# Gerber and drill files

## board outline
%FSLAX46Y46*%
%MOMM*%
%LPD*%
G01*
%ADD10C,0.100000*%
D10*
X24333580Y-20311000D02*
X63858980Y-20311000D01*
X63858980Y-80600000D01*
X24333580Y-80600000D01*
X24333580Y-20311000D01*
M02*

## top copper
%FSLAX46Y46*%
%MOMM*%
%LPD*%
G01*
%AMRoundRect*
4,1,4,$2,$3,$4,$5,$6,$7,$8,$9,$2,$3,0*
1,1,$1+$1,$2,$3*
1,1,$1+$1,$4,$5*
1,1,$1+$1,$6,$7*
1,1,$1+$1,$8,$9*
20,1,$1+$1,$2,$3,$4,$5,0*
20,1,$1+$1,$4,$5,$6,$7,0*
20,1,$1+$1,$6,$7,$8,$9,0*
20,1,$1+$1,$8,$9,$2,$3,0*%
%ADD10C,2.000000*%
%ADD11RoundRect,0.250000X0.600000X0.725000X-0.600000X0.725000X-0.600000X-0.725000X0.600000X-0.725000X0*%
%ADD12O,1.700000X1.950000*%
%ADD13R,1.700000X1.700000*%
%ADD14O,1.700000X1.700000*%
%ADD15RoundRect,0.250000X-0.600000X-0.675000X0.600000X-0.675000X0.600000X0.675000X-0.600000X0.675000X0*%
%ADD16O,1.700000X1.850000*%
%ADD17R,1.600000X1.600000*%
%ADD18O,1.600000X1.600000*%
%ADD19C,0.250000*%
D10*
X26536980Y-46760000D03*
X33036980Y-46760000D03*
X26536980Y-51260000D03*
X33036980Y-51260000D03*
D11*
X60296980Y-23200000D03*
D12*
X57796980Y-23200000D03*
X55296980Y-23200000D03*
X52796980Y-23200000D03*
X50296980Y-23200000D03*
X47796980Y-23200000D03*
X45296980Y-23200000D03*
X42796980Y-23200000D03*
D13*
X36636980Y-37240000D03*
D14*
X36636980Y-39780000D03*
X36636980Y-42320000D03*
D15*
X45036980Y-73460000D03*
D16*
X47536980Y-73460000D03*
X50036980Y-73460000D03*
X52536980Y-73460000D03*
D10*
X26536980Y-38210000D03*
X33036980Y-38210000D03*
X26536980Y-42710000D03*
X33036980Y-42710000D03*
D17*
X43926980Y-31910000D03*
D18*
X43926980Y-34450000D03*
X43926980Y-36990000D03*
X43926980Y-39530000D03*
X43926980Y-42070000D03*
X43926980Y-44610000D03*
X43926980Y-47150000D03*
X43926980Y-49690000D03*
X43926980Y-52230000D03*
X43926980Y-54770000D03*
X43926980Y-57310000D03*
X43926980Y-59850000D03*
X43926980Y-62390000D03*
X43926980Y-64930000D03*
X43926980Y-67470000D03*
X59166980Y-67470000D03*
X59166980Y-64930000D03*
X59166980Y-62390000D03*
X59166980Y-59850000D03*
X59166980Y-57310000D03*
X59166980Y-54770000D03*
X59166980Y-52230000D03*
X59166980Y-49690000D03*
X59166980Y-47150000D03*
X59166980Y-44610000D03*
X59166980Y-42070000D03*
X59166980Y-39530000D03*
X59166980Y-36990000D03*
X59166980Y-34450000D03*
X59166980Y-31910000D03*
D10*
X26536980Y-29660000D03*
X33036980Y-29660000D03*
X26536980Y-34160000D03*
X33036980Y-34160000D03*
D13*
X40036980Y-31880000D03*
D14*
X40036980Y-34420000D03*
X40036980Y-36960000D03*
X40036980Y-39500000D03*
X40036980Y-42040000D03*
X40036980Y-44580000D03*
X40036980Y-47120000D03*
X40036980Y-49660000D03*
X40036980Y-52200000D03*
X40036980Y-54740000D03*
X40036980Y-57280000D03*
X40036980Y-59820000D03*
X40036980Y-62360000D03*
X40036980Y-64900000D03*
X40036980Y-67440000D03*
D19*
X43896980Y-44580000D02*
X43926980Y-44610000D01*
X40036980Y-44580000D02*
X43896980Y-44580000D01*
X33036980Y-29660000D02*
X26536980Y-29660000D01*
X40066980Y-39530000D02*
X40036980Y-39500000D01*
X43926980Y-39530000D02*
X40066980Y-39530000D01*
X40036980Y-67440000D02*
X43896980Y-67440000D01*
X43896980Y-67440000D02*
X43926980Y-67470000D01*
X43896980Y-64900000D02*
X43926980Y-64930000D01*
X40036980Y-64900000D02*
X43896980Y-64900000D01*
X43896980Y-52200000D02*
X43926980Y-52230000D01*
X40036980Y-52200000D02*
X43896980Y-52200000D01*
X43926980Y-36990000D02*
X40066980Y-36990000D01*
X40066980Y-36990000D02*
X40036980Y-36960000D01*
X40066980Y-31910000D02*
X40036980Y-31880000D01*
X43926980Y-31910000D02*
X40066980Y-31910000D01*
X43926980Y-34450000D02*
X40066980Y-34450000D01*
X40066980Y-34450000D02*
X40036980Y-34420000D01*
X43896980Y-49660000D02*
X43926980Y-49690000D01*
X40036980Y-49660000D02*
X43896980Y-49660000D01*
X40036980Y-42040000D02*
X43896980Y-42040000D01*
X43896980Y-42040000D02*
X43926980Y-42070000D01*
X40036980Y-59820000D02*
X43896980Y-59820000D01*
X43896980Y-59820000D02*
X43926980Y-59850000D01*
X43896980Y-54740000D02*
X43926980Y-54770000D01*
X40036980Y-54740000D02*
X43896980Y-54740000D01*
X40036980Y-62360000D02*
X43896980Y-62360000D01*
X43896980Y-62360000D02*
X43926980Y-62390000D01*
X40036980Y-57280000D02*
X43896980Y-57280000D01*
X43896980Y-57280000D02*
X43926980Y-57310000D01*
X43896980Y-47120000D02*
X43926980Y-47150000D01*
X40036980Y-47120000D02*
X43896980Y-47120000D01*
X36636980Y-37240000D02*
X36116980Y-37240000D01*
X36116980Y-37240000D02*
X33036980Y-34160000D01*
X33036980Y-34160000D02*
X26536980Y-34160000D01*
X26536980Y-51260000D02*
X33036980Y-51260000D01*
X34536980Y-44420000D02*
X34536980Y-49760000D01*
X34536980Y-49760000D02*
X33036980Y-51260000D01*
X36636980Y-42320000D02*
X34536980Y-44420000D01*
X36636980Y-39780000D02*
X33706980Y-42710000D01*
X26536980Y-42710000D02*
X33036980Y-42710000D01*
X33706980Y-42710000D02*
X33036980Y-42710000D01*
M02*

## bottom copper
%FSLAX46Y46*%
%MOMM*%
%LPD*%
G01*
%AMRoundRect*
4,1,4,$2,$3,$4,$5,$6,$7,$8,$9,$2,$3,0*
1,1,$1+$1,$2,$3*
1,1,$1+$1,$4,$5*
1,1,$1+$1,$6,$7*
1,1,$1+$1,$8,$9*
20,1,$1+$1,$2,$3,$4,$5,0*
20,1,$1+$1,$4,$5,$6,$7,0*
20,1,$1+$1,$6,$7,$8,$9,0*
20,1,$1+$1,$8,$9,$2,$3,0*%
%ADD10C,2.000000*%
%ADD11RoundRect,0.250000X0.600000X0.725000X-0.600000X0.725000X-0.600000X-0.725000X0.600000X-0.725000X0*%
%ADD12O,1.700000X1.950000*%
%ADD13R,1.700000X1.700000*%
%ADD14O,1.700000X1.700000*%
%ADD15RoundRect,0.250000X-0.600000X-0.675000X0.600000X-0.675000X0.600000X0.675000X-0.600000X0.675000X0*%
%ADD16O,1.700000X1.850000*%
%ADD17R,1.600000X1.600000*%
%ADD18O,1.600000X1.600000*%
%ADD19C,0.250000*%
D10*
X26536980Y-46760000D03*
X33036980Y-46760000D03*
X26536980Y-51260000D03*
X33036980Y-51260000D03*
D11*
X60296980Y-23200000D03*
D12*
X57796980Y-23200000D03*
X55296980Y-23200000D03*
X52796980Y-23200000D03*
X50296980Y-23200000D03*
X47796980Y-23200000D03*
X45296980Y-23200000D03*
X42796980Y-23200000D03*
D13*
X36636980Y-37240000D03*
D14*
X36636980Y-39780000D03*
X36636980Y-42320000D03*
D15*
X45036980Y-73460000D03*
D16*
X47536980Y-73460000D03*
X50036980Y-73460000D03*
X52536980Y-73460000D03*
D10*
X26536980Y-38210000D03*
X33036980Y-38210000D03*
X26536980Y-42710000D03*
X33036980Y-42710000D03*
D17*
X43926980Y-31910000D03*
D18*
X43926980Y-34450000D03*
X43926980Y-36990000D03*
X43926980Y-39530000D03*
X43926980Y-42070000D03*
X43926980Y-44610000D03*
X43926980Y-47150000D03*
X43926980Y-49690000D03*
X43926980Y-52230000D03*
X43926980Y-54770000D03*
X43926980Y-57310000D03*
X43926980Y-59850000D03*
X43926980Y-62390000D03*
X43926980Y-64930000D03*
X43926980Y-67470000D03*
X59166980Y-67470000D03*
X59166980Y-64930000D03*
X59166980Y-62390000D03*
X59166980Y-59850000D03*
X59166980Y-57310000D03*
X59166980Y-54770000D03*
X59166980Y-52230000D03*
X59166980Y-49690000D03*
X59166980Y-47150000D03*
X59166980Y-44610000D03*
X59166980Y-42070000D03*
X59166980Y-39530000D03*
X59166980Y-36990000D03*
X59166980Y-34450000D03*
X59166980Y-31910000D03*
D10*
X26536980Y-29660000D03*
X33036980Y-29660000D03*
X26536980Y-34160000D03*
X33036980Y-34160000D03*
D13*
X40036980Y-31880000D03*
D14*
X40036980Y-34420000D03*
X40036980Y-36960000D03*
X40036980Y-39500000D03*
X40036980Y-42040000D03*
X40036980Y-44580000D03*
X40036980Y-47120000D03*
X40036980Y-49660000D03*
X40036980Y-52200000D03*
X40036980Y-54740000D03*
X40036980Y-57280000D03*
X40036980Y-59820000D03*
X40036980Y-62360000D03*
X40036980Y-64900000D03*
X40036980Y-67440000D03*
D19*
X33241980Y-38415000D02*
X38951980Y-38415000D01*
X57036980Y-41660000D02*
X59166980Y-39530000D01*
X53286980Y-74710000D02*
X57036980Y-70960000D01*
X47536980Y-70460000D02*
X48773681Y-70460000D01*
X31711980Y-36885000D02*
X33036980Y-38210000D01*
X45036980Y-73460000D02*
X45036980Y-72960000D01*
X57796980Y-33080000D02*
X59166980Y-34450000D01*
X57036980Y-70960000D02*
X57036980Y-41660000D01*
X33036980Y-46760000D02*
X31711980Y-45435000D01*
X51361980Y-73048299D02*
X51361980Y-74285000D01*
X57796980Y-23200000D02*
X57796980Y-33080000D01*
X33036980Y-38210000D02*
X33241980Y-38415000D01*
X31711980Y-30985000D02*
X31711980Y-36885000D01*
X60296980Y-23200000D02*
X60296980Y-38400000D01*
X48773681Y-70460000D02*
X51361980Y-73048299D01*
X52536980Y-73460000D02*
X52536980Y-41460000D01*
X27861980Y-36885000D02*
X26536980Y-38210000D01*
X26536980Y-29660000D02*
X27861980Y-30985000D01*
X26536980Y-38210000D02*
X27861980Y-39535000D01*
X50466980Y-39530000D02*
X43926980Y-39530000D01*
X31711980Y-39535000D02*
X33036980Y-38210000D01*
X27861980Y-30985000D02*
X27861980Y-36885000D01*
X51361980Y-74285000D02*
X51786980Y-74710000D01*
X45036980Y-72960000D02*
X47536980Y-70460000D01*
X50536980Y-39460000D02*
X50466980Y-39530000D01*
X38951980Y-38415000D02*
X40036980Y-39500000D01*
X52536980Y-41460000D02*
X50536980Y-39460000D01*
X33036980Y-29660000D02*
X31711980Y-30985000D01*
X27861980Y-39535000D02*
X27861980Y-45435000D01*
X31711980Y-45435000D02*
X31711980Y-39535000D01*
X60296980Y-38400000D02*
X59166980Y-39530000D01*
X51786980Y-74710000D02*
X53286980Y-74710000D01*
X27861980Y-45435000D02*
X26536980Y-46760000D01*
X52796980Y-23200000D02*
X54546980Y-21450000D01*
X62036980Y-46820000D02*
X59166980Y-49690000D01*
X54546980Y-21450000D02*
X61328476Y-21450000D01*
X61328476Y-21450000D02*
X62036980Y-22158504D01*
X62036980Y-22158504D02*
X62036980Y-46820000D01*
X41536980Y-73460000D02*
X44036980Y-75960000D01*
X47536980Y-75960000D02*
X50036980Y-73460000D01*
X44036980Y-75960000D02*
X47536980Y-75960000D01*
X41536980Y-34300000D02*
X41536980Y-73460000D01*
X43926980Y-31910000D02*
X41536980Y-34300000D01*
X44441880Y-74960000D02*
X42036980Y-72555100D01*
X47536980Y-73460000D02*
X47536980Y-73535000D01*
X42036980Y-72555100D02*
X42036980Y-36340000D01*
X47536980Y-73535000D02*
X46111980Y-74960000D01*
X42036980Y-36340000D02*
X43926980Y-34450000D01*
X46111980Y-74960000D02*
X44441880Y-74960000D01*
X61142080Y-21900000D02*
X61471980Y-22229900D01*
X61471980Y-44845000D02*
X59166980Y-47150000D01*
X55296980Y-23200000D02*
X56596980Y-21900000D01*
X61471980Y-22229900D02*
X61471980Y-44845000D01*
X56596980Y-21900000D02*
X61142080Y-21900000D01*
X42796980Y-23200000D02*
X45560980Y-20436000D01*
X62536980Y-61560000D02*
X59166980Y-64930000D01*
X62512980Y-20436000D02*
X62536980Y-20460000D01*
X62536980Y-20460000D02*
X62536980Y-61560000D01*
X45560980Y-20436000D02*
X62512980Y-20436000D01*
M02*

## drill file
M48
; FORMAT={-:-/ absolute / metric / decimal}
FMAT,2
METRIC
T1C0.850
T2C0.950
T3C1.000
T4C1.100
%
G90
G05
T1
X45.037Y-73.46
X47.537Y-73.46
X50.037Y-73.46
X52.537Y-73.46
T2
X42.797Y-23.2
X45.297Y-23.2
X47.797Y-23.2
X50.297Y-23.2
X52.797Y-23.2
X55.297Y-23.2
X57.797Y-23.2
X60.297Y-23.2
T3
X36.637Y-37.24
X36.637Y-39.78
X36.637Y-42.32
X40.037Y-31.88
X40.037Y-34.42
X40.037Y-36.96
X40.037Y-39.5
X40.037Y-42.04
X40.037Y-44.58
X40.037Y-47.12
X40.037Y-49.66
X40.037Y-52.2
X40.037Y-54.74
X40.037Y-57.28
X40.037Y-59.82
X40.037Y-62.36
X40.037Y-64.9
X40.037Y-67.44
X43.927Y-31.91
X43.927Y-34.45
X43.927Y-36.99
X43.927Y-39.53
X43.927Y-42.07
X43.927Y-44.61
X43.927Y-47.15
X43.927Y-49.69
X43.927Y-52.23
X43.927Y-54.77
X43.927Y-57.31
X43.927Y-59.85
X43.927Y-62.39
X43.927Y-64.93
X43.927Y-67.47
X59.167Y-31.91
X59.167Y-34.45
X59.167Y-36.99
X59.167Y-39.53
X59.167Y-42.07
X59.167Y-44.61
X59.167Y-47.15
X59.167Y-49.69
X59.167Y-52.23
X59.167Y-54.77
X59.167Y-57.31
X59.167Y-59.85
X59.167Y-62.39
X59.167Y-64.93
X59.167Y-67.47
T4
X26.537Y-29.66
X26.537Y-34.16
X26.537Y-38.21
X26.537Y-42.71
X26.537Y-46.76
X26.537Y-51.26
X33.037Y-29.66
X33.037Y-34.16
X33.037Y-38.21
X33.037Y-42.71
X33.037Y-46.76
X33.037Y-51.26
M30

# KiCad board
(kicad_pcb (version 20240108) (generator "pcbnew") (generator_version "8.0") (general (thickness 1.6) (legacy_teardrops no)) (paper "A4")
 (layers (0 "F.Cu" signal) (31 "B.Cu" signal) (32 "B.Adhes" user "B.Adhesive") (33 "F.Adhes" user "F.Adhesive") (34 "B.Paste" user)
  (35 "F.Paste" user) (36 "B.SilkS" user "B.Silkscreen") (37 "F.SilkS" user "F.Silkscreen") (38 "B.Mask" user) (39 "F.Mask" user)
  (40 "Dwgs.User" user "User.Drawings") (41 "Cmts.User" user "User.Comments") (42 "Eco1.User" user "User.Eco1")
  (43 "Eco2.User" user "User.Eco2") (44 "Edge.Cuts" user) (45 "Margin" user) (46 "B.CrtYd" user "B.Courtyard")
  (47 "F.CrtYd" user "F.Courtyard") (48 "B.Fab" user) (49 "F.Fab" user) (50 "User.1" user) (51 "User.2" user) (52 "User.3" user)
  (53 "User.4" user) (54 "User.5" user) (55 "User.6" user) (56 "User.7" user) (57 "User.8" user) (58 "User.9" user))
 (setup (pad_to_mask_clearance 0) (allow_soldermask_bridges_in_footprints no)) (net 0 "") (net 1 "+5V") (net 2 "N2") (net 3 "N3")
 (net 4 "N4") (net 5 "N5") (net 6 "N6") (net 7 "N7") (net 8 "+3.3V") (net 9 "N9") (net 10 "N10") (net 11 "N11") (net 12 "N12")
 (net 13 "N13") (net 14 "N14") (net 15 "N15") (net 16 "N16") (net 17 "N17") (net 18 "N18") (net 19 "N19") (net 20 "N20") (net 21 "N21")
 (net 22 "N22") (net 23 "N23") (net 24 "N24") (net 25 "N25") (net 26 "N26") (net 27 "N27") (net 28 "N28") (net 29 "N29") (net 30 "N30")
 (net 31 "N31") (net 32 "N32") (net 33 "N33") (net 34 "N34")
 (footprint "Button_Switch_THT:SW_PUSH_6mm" (layer "F.Cu") (at 26.53698 46.76)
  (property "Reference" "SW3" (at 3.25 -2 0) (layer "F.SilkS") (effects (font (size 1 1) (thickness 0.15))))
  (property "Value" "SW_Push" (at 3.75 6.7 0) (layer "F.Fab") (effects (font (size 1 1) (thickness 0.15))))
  (pad "1" thru_hole circle (at 0 0 90) (size 2 2) (drill 1.1) (layers "*.Cu" "*.Mask") (remove_unused_layers no) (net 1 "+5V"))
  (pad "1" thru_hole circle (at 6.5 0 90) (size 2 2) (drill 1.1) (layers "*.Cu" "*.Mask") (remove_unused_layers no) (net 1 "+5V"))
  (pad "2" thru_hole circle (at 0 4.5 90) (size 2 2) (drill 1.1) (layers "*.Cu" "*.Mask") (remove_unused_layers no) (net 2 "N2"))
  (pad "2" thru_hole circle (at 6.5 4.5 90) (size 2 2) (drill 1.1) (layers "*.Cu" "*.Mask") (remove_unused_layers no) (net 2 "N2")))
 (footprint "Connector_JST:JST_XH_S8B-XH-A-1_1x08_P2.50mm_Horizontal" (layer "F.Cu") (at 60.29698 23.2 180)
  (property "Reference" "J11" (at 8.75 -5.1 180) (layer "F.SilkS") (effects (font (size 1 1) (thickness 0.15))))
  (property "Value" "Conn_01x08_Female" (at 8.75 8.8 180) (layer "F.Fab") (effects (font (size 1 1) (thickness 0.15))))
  (pad "1" thru_hole roundrect (at 0 0 180) (size 1.7 1.95) (drill 0.95) (layers "*.Cu" "*.Mask") (remove_unused_layers no)
   (roundrect_rratio 0.147059) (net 1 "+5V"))
  (pad "2" thru_hole oval (at 2.5 0 180) (size 1.7 1.95) (drill 0.95) (layers "*.Cu" "*.Mask") (remove_unused_layers no) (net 1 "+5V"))
  (pad "3" thru_hole oval (at 5 0 180) (size 1.7 1.95) (drill 0.95) (layers "*.Cu" "*.Mask") (remove_unused_layers no) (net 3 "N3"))
  (pad "4" thru_hole oval (at 7.5 0 180) (size 1.7 1.95) (drill 0.95) (layers "*.Cu" "*.Mask") (remove_unused_layers no) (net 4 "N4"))
  (pad "5" thru_hole oval (at 10 0 180) (size 1.7 1.95) (drill 0.95) (layers "*.Cu" "*.Mask") (remove_unused_layers no) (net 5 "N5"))
  (pad "6" thru_hole oval (at 12.5 0 180) (size 1.7 1.95) (drill 0.95) (layers "*.Cu" "*.Mask") (remove_unused_layers no) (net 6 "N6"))
  (pad "7" thru_hole oval (at 15 0 180) (size 1.7 1.95) (drill 0.95) (layers "*.Cu" "*.Mask") (remove_unused_layers no) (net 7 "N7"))
  (pad "8" thru_hole oval (at 17.5 0 180) (size 1.7 1.95) (drill 0.95) (layers "*.Cu" "*.Mask") (remove_unused_layers no) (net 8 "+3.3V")))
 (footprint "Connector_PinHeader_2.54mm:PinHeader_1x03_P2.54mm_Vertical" (layer "F.Cu") (at 36.63698 37.24)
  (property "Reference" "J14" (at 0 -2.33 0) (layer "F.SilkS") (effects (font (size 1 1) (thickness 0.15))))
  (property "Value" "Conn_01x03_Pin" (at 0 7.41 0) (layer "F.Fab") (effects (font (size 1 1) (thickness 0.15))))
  (pad "1" thru_hole rect (at 0 0) (size 1.7 1.7) (drill 1) (layers "*.Cu" "*.Mask") (remove_unused_layers no) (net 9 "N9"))
  (pad "2" thru_hole oval (at 0 2.54) (size 1.7 1.7) (drill 1) (layers "*.Cu" "*.Mask") (remove_unused_layers no) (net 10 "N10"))
  (pad "3" thru_hole oval (at 0 5.08) (size 1.7 1.7) (drill 1) (layers "*.Cu" "*.Mask") (remove_unused_layers no) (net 2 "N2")))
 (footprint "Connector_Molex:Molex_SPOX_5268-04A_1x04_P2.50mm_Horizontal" (layer "F.Cu") (at 45.03698 73.46)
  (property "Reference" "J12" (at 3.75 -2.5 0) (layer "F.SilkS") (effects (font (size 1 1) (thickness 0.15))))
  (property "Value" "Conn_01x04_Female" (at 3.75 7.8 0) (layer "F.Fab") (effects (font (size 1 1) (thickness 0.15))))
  (pad "1" thru_hole roundrect (at 0 0) (size 1.7 1.85) (drill 0.85) (layers "*.Cu" "*.Mask") (remove_unused_layers no)
   (roundrect_rratio 0.147059) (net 1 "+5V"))
  (pad "2" thru_hole oval (at 2.5 0) (size 1.7 1.85) (drill 0.85) (layers "*.Cu" "*.Mask") (remove_unused_layers no) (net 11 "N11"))
  (pad "3" thru_hole oval (at 5 0) (size 1.7 1.85) (drill 0.85) (layers "*.Cu" "*.Mask") (remove_unused_layers no) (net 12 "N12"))
  (pad "4" thru_hole oval (at 7.5 0) (size 1.7 1.85) (drill 0.85) (layers "*.Cu" "*.Mask") (remove_unused_layers no) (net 1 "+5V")))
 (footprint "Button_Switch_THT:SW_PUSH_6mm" (layer "F.Cu") (at 26.53698 38.21)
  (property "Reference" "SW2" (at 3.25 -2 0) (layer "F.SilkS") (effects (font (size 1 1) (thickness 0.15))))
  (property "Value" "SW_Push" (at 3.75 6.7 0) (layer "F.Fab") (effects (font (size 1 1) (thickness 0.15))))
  (pad "1" thru_hole circle (at 0 0 90) (size 2 2) (drill 1.1) (layers "*.Cu" "*.Mask") (remove_unused_layers no) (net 1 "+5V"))
  (pad "1" thru_hole circle (at 6.5 0 90) (size 2 2) (drill 1.1) (layers "*.Cu" "*.Mask") (remove_unused_layers no) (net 1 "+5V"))
  (pad "2" thru_hole circle (at 0 4.5 90) (size 2 2) (drill 1.1) (layers "*.Cu" "*.Mask") (remove_unused_layers no) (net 10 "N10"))
  (pad "2" thru_hole circle (at 6.5 4.5 90) (size 2 2) (drill 1.1) (layers "*.Cu" "*.Mask") (remove_unused_layers no) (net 10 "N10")))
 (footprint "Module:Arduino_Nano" (layer "F.Cu") (at 43.92698 31.91)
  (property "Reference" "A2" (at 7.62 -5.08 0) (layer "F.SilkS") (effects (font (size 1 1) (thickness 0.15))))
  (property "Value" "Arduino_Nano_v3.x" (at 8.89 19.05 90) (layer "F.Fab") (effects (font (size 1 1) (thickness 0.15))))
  (pad "1" thru_hole rect (at 0 0) (size 1.6 1.6) (drill 1) (layers "*.Cu" "*.Mask") (remove_unused_layers no) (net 12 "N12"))
  (pad "2" thru_hole oval (at 0 2.54) (size 1.6 1.6) (drill 1) (layers "*.Cu" "*.Mask") (remove_unused_layers no) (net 11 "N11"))
  (pad "3" thru_hole oval (at 0 5.08) (size 1.6 1.6) (drill 1) (layers "*.Cu" "*.Mask") (remove_unused_layers no) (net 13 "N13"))
  (pad "4" thru_hole oval (at 0 7.62) (size 1.6 1.6) (drill 1) (layers "*.Cu" "*.Mask") (remove_unused_layers no) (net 1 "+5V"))
  (pad "5" thru_hole oval (at 0 10.16) (size 1.6 1.6) (drill 1) (layers "*.Cu" "*.Mask") (remove_unused_layers no) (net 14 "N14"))
  (pad "6" thru_hole oval (at 0 12.7) (size 1.6 1.6) (drill 1) (layers "*.Cu" "*.Mask") (remove_unused_layers no) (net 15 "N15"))
  (pad "7" thru_hole oval (at 0 15.24) (size 1.6 1.6) (drill 1) (layers "*.Cu" "*.Mask") (remove_unused_layers no) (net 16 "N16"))
  (pad "8" thru_hole oval (at 0 17.78) (size 1.6 1.6) (drill 1) (layers "*.Cu" "*.Mask") (remove_unused_layers no) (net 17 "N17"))
  (pad "9" thru_hole oval (at 0 20.32) (size 1.6 1.6) (drill 1) (layers "*.Cu" "*.Mask") (remove_unused_layers no) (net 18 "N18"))
  (pad "10" thru_hole oval (at 0 22.86) (size 1.6 1.6) (drill 1) (layers "*.Cu" "*.Mask") (remove_unused_layers no) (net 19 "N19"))
  (pad "11" thru_hole oval (at 0 25.4) (size 1.6 1.6) (drill 1) (layers "*.Cu" "*.Mask") (remove_unused_layers no) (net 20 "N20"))
  (pad "12" thru_hole oval (at 0 27.94) (size 1.6 1.6) (drill 1) (layers "*.Cu" "*.Mask") (remove_unused_layers no) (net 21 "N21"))
  (pad "13" thru_hole oval (at 0 30.48) (size 1.6 1.6) (drill 1) (layers "*.Cu" "*.Mask") (remove_unused_layers no) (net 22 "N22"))
  (pad "14" thru_hole oval (at 0 33.02) (size 1.6 1.6) (drill 1) (layers "*.Cu" "*.Mask") (remove_unused_layers no) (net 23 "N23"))
  (pad "15" thru_hole oval (at 0 35.56) (size 1.6 1.6) (drill 1) (layers "*.Cu" "*.Mask") (remove_unused_layers no) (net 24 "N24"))
  (pad "16" thru_hole oval (at 15.24 35.56) (size 1.6 1.6) (drill 1) (layers "*.Cu" "*.Mask") (remove_unused_layers no) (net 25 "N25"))
  (pad "17" thru_hole oval (at 15.24 33.02) (size 1.6 1.6) (drill 1) (layers "*.Cu" "*.Mask") (remove_unused_layers no) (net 8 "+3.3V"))
  (pad "18" thru_hole oval (at 15.24 30.48) (size 1.6 1.6) (drill 1) (layers "*.Cu" "*.Mask") (remove_unused_layers no) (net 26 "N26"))
  (pad "19" thru_hole oval (at 15.24 27.94) (size 1.6 1.6) (drill 1) (layers "*.Cu" "*.Mask") (remove_unused_layers no) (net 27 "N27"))
  (pad "20" thru_hole oval (at 15.24 25.4) (size 1.6 1.6) (drill 1) (layers "*.Cu" "*.Mask") (remove_unused_layers no) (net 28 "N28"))
  (pad "21" thru_hole oval (at 15.24 22.86) (size 1.6 1.6) (drill 1) (layers "*.Cu" "*.Mask") (remove_unused_layers no) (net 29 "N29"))
  (pad "22" thru_hole oval (at 15.24 20.32) (size 1.6 1.6) (drill 1) (layers "*.Cu" "*.Mask") (remove_unused_layers no) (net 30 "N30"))
  (pad "23" thru_hole oval (at 15.24 17.78) (size 1.6 1.6) (drill 1) (layers "*.Cu" "*.Mask") (remove_unused_layers no) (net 4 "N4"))
  (pad "24" thru_hole oval (at 15.24 15.24) (size 1.6 1.6) (drill 1) (layers "*.Cu" "*.Mask") (remove_unused_layers no) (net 3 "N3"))
  (pad "25" thru_hole oval (at 15.24 12.7) (size 1.6 1.6) (drill 1) (layers "*.Cu" "*.Mask") (remove_unused_layers no) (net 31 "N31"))
  (pad "26" thru_hole oval (at 15.24 10.16) (size 1.6 1.6) (drill 1) (layers "*.Cu" "*.Mask") (remove_unused_layers no) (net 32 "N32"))
  (pad "27" thru_hole oval (at 15.24 7.62) (size 1.6 1.6) (drill 1) (layers "*.Cu" "*.Mask") (remove_unused_layers no) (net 1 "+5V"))
  (pad "28" thru_hole oval (at 15.24 5.08) (size 1.6 1.6) (drill 1) (layers "*.Cu" "*.Mask") (remove_unused_layers no) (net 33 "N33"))
  (pad "29" thru_hole oval (at 15.24 2.54) (size 1.6 1.6) (drill 1) (layers "*.Cu" "*.Mask") (remove_unused_layers no) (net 1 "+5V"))
  (pad "30" thru_hole oval (at 15.24 0) (size 1.6 1.6) (drill 1) (layers "*.Cu" "*.Mask") (remove_unused_layers no) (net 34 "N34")))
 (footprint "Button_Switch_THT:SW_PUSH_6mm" (layer "F.Cu") (at 26.53698 29.66)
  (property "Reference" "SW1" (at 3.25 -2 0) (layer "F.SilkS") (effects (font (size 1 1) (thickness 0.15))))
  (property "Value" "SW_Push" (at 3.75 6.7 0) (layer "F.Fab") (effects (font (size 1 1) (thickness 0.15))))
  (pad "1" thru_hole circle (at 0 0 90) (size 2 2) (drill 1.1) (layers "*.Cu" "*.Mask") (remove_unused_layers no) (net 1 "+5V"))
  (pad "1" thru_hole circle (at 6.5 0 90) (size 2 2) (drill 1.1) (layers "*.Cu" "*.Mask") (remove_unused_layers no) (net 1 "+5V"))
  (pad "2" thru_hole circle (at 0 4.5 90) (size 2 2) (drill 1.1) (layers "*.Cu" "*.Mask") (remove_unused_layers no) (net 9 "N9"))
  (pad "2" thru_hole circle (at 6.5 4.5 90) (size 2 2) (drill 1.1) (layers "*.Cu" "*.Mask") (remove_unused_layers no) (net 9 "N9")))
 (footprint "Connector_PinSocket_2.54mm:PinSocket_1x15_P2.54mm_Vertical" (layer "F.Cu") (at 40.03698 31.88)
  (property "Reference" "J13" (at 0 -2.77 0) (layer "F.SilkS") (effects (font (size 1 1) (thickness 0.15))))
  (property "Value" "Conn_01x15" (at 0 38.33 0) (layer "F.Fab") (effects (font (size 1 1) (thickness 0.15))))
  (pad "1" thru_hole rect (at 0 0) (size 1.7 1.7) (drill 1) (layers "*.Cu" "*.Mask") (remove_unused_layers no) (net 12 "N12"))
  (pad "2" thru_hole oval (at 0 2.54) (size 1.7 1.7) (drill 1) (layers "*.Cu" "*.Mask") (remove_unused_layers no) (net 11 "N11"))
  (pad "3" thru_hole oval (at 0 5.08) (size 1.7 1.7) (drill 1) (layers "*.Cu" "*.Mask") (remove_unused_layers no) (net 13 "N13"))
  (pad "4" thru_hole oval (at 0 7.62) (size 1.7 1.7) (drill 1) (layers "*.Cu" "*.Mask") (remove_unused_layers no) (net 1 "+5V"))
  (pad "5" thru_hole oval (at 0 10.16) (size 1.7 1.7) (drill 1) (layers "*.Cu" "*.Mask") (remove_unused_layers no) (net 14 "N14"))
  (pad "6" thru_hole oval (at 0 12.7) (size 1.7 1.7) (drill 1) (layers "*.Cu" "*.Mask") (remove_unused_layers no) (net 15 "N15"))
  (pad "7" thru_hole oval (at 0 15.24) (size 1.7 1.7) (drill 1) (layers "*.Cu" "*.Mask") (remove_unused_layers no) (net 16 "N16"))
  (pad "8" thru_hole oval (at 0 17.78) (size 1.7 1.7) (drill 1) (layers "*.Cu" "*.Mask") (remove_unused_layers no) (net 17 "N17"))
  (pad "9" thru_hole oval (at 0 20.32) (size 1.7 1.7) (drill 1) (layers "*.Cu" "*.Mask") (remove_unused_layers no) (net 18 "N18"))
  (pad "10" thru_hole oval (at 0 22.86) (size 1.7 1.7) (drill 1) (layers "*.Cu" "*.Mask") (remove_unused_layers no) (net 19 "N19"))
  (pad "11" thru_hole oval (at 0 25.4) (size 1.7 1.7) (drill 1) (layers "*.Cu" "*.Mask") (remove_unused_layers no) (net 20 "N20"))
  (pad "12" thru_hole oval (at 0 27.94) (size 1.7 1.7) (drill 1) (layers "*.Cu" "*.Mask") (remove_unused_layers no) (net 21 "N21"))
  (pad "13" thru_hole oval (at 0 30.48) (size 1.7 1.7) (drill 1) (layers "*.Cu" "*.Mask") (remove_unused_layers no) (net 22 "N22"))
  (pad "14" thru_hole oval (at 0 33.02) (size 1.7 1.7) (drill 1) (layers "*.Cu" "*.Mask") (remove_unused_layers no) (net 23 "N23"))
  (pad "15" thru_hole oval (at 0 35.56) (size 1.7 1.7) (drill 1) (layers "*.Cu" "*.Mask") (remove_unused_layers no) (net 24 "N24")))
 (gr_rect (start 24.33358 20.311) (end 63.85898 80.6) (stroke (width 0.1) (type default)) (fill none) (layer "Edge.Cuts"))
 (segment (start 43.89698 44.58) (end 43.92698 44.61) (width 0.25) (layer "F.Cu") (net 15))
 (segment (start 40.03698 44.58) (end 43.89698 44.58) (width 0.25) (layer "F.Cu") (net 15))
 (segment (start 33.03698 29.66) (end 26.53698 29.66) (width 0.25) (layer "F.Cu") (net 1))
 (segment (start 40.06698 39.53) (end 40.03698 39.5) (width 0.25) (layer "F.Cu") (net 1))
 (segment (start 43.92698 39.53) (end 40.06698 39.53) (width 0.25) (layer "F.Cu") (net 1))
 (segment (start 33.24198 38.415) (end 38.95198 38.415) (width 0.25) (layer "B.Cu") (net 1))
 (segment (start 57.03698 41.66) (end 59.16698 39.53) (width 0.25) (layer "B.Cu") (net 1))
 (segment (start 53.28698 74.71) (end 57.03698 70.96) (width 0.25) (layer "B.Cu") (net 1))
 (segment (start 47.53698 70.46) (end 48.773681 70.46) (width 0.25) (layer "B.Cu") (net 1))
 (segment (start 31.71198 36.885) (end 33.03698 38.21) (width 0.25) (layer "B.Cu") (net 1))
 (segment (start 45.03698 73.46) (end 45.03698 72.96) (width 0.25) (layer "B.Cu") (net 1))
 (segment (start 57.79698 33.08) (end 59.16698 34.45) (width 0.25) (layer "B.Cu") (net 1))
 (segment (start 57.03698 70.96) (end 57.03698 41.66) (width 0.25) (layer "B.Cu") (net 1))
 (segment (start 33.03698 46.76) (end 31.71198 45.435) (width 0.25) (layer "B.Cu") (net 1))
 (segment (start 51.36198 73.048299) (end 51.36198 74.285) (width 0.25) (layer "B.Cu") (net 1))
 (segment (start 57.79698 23.2) (end 57.79698 33.08) (width 0.25) (layer "B.Cu") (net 1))
 (segment (start 33.03698 38.21) (end 33.24198 38.415) (width 0.25) (layer "B.Cu") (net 1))
 (segment (start 31.71198 30.985) (end 31.71198 36.885) (width 0.25) (layer "B.Cu") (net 1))
 (segment (start 60.29698 23.2) (end 60.29698 38.4) (width 0.25) (layer "B.Cu") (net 1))
 (segment (start 48.773681 70.46) (end 51.36198 73.048299) (width 0.25) (layer "B.Cu") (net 1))
 (segment (start 52.53698 73.46) (end 52.53698 41.46) (width 0.25) (layer "B.Cu") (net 1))
 (segment (start 27.86198 36.885) (end 26.53698 38.21) (width 0.25) (layer "B.Cu") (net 1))
 (segment (start 26.53698 29.66) (end 27.86198 30.985) (width 0.25) (layer "B.Cu") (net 1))
 (segment (start 26.53698 38.21) (end 27.86198 39.535) (width 0.25) (layer "B.Cu") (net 1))
 (segment (start 50.46698 39.53) (end 43.92698 39.53) (width 0.25) (layer "B.Cu") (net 1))
 (segment (start 31.71198 39.535) (end 33.03698 38.21) (width 0.25) (layer "B.Cu") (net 1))
 (segment (start 27.86198 30.985) (end 27.86198 36.885) (width 0.25) (layer "B.Cu") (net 1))
 (segment (start 51.36198 74.285) (end 51.78698 74.71) (width 0.25) (layer "B.Cu") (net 1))
 (segment (start 45.03698 72.96) (end 47.53698 70.46) (width 0.25) (layer "B.Cu") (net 1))
 (segment (start 50.53698 39.46) (end 50.46698 39.53) (width 0.25) (layer "B.Cu") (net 1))
 (segment (start 38.95198 38.415) (end 40.03698 39.5) (width 0.25) (layer "B.Cu") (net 1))
 (segment (start 52.53698 41.46) (end 50.53698 39.46) (width 0.25) (layer "B.Cu") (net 1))
 (segment (start 33.03698 29.66) (end 31.71198 30.985) (width 0.25) (layer "B.Cu") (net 1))
 (segment (start 27.86198 39.535) (end 27.86198 45.435) (width 0.25) (layer "B.Cu") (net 1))
 (segment (start 31.71198 45.435) (end 31.71198 39.535) (width 0.25) (layer "B.Cu") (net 1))
 (segment (start 60.29698 38.4) (end 59.16698 39.53) (width 0.25) (layer "B.Cu") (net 1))
 (segment (start 51.78698 74.71) (end 53.28698 74.71) (width 0.25) (layer "B.Cu") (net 1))
 (segment (start 27.86198 45.435) (end 26.53698 46.76) (width 0.25) (layer "B.Cu") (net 1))
 (segment (start 52.79698 23.2) (end 54.54698 21.45) (width 0.25) (layer "B.Cu") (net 4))
 (segment (start 62.03698 46.82) (end 59.16698 49.69) (width 0.25) (layer "B.Cu") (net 4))
 (segment (start 54.54698 21.45) (end 61.328476 21.45) (width 0.25) (layer "B.Cu") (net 4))
 (segment (start 61.328476 21.45) (end 62.03698 22.158504) (width 0.25) (layer "B.Cu") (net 4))
 (segment (start 62.03698 22.158504) (end 62.03698 46.82) (width 0.25) (layer "B.Cu") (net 4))
 (segment (start 40.03698 67.44) (end 43.89698 67.44) (width 0.25) (layer "F.Cu") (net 24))
 (segment (start 43.89698 67.44) (end 43.92698 67.47) (width 0.25) (layer "F.Cu") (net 24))
 (segment (start 43.89698 64.9) (end 43.92698 64.93) (width 0.25) (layer "F.Cu") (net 23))
 (segment (start 40.03698 64.9) (end 43.89698 64.9) (width 0.25) (layer "F.Cu") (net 23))
 (segment (start 43.89698 52.2) (end 43.92698 52.23) (width 0.25) (layer "F.Cu") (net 18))
 (segment (start 40.03698 52.2) (end 43.89698 52.2) (width 0.25) (layer "F.Cu") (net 18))
 (segment (start 43.92698 36.99) (end 40.06698 36.99) (width 0.25) (layer "F.Cu") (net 13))
 (segment (start 40.06698 36.99) (end 40.03698 36.96) (width 0.25) (layer "F.Cu") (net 13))
 (segment (start 40.06698 31.91) (end 40.03698 31.88) (width 0.25) (layer "F.Cu") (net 12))
 (segment (start 43.92698 31.91) (end 40.06698 31.91) (width 0.25) (layer "F.Cu") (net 12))
 (segment (start 41.53698 73.46) (end 44.03698 75.96) (width 0.25) (layer "B.Cu") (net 12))
 (segment (start 47.53698 75.96) (end 50.03698 73.46) (width 0.25) (layer "B.Cu") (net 12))
 (segment (start 44.03698 75.96) (end 47.53698 75.96) (width 0.25) (layer "B.Cu") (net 12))
 (segment (start 41.53698 34.3) (end 41.53698 73.46) (width 0.25) (layer "B.Cu") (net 12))
 (segment (start 43.92698 31.91) (end 41.53698 34.3) (width 0.25) (layer "B.Cu") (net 12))
 (segment (start 43.92698 34.45) (end 40.06698 34.45) (width 0.25) (layer "F.Cu") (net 11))
 (segment (start 40.06698 34.45) (end 40.03698 34.42) (width 0.25) (layer "F.Cu") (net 11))
 (segment (start 44.44188 74.96) (end 42.03698 72.5551) (width 0.25) (layer "B.Cu") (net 11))
 (segment (start 47.53698 73.46) (end 47.53698 73.535) (width 0.25) (layer "B.Cu") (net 11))
 (segment (start 42.03698 72.5551) (end 42.03698 36.34) (width 0.25) (layer "B.Cu") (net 11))
 (segment (start 47.53698 73.535) (end 46.11198 74.96) (width 0.25) (layer "B.Cu") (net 11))
 (segment (start 42.03698 36.34) (end 43.92698 34.45) (width 0.25) (layer "B.Cu") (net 11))
 (segment (start 46.11198 74.96) (end 44.44188 74.96) (width 0.25) (layer "B.Cu") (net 11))
 (segment (start 43.89698 49.66) (end 43.92698 49.69) (width 0.25) (layer "F.Cu") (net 17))
 (segment (start 40.03698 49.66) (end 43.89698 49.66) (width 0.25) (layer "F.Cu") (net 17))
 (segment (start 40.03698 42.04) (end 43.89698 42.04) (width 0.25) (layer "F.Cu") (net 14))
 (segment (start 43.89698 42.04) (end 43.92698 42.07) (width 0.25) (layer "F.Cu") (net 14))
 (segment (start 40.03698 59.82) (end 43.89698 59.82) (width 0.25) (layer "F.Cu") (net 21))
 (segment (start 43.89698 59.82) (end 43.92698 59.85) (width 0.25) (layer "F.Cu") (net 21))
 (segment (start 61.14208 21.9) (end 61.47198 22.2299) (width 0.25) (layer "B.Cu") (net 3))
 (segment (start 61.47198 44.845) (end 59.16698 47.15) (width 0.25) (layer "B.Cu") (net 3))
 (segment (start 55.29698 23.2) (end 56.59698 21.9) (width 0.25) (layer "B.Cu") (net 3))
 (segment (start 61.47198 22.2299) (end 61.47198 44.845) (width 0.25) (layer "B.Cu") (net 3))
 (segment (start 56.59698 21.9) (end 61.14208 21.9) (width 0.25) (layer "B.Cu") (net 3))
 (segment (start 43.89698 54.74) (end 43.92698 54.77) (width 0.25) (layer "F.Cu") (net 19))
 (segment (start 40.03698 54.74) (end 43.89698 54.74) (width 0.25) (layer "F.Cu") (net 19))
 (segment (start 40.03698 62.36) (end 43.89698 62.36) (width 0.25) (layer "F.Cu") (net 22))
 (segment (start 43.89698 62.36) (end 43.92698 62.39) (width 0.25) (layer "F.Cu") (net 22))
 (segment (start 42.79698 23.2) (end 45.56098 20.436) (width 0.25) (layer "B.Cu") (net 8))
 (segment (start 62.53698 61.56) (end 59.16698 64.93) (width 0.25) (layer "B.Cu") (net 8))
 (segment (start 62.51298 20.436) (end 62.53698 20.46) (width 0.25) (layer "B.Cu") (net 8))
 (segment (start 62.53698 20.46) (end 62.53698 61.56) (width 0.25) (layer "B.Cu") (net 8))
 (segment (start 45.56098 20.436) (end 62.51298 20.436) (width 0.25) (layer "B.Cu") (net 8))
 (segment (start 40.03698 57.28) (end 43.89698 57.28) (width 0.25) (layer "F.Cu") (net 20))
 (segment (start 43.89698 57.28) (end 43.92698 57.31) (width 0.25) (layer "F.Cu") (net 20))
 (segment (start 43.89698 47.12) (end 43.92698 47.15) (width 0.25) (layer "F.Cu") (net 16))
 (segment (start 40.03698 47.12) (end 43.89698 47.12) (width 0.25) (layer "F.Cu") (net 16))
 (segment (start 36.63698 37.24) (end 36.11698 37.24) (width 0.25) (layer "F.Cu") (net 9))
 (segment (start 36.11698 37.24) (end 33.03698 34.16) (width 0.25) (layer "F.Cu") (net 9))
 (segment (start 33.03698 34.16) (end 26.53698 34.16) (width 0.25) (layer "F.Cu") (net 9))
 (segment (start 26.53698 51.26) (end 33.03698 51.26) (width 0.25) (layer "F.Cu") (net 2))
 (segment (start 34.53698 44.42) (end 34.53698 49.76) (width 0.25) (layer "F.Cu") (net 2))
 (segment (start 34.53698 49.76) (end 33.03698 51.26) (width 0.25) (layer "F.Cu") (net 2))
 (segment (start 36.63698 42.32) (end 34.53698 44.42) (width 0.25) (layer "F.Cu") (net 2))
 (segment (start 36.63698 39.78) (end 33.70698 42.71) (width 0.25) (layer "F.Cu") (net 10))
 (segment (start 26.53698 42.71) (end 33.03698 42.71) (width 0.25) (layer "F.Cu") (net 10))
 (segment (start 33.70698 42.71) (end 33.03698 42.71) (width 0.25) (layer "F.Cu") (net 10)))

